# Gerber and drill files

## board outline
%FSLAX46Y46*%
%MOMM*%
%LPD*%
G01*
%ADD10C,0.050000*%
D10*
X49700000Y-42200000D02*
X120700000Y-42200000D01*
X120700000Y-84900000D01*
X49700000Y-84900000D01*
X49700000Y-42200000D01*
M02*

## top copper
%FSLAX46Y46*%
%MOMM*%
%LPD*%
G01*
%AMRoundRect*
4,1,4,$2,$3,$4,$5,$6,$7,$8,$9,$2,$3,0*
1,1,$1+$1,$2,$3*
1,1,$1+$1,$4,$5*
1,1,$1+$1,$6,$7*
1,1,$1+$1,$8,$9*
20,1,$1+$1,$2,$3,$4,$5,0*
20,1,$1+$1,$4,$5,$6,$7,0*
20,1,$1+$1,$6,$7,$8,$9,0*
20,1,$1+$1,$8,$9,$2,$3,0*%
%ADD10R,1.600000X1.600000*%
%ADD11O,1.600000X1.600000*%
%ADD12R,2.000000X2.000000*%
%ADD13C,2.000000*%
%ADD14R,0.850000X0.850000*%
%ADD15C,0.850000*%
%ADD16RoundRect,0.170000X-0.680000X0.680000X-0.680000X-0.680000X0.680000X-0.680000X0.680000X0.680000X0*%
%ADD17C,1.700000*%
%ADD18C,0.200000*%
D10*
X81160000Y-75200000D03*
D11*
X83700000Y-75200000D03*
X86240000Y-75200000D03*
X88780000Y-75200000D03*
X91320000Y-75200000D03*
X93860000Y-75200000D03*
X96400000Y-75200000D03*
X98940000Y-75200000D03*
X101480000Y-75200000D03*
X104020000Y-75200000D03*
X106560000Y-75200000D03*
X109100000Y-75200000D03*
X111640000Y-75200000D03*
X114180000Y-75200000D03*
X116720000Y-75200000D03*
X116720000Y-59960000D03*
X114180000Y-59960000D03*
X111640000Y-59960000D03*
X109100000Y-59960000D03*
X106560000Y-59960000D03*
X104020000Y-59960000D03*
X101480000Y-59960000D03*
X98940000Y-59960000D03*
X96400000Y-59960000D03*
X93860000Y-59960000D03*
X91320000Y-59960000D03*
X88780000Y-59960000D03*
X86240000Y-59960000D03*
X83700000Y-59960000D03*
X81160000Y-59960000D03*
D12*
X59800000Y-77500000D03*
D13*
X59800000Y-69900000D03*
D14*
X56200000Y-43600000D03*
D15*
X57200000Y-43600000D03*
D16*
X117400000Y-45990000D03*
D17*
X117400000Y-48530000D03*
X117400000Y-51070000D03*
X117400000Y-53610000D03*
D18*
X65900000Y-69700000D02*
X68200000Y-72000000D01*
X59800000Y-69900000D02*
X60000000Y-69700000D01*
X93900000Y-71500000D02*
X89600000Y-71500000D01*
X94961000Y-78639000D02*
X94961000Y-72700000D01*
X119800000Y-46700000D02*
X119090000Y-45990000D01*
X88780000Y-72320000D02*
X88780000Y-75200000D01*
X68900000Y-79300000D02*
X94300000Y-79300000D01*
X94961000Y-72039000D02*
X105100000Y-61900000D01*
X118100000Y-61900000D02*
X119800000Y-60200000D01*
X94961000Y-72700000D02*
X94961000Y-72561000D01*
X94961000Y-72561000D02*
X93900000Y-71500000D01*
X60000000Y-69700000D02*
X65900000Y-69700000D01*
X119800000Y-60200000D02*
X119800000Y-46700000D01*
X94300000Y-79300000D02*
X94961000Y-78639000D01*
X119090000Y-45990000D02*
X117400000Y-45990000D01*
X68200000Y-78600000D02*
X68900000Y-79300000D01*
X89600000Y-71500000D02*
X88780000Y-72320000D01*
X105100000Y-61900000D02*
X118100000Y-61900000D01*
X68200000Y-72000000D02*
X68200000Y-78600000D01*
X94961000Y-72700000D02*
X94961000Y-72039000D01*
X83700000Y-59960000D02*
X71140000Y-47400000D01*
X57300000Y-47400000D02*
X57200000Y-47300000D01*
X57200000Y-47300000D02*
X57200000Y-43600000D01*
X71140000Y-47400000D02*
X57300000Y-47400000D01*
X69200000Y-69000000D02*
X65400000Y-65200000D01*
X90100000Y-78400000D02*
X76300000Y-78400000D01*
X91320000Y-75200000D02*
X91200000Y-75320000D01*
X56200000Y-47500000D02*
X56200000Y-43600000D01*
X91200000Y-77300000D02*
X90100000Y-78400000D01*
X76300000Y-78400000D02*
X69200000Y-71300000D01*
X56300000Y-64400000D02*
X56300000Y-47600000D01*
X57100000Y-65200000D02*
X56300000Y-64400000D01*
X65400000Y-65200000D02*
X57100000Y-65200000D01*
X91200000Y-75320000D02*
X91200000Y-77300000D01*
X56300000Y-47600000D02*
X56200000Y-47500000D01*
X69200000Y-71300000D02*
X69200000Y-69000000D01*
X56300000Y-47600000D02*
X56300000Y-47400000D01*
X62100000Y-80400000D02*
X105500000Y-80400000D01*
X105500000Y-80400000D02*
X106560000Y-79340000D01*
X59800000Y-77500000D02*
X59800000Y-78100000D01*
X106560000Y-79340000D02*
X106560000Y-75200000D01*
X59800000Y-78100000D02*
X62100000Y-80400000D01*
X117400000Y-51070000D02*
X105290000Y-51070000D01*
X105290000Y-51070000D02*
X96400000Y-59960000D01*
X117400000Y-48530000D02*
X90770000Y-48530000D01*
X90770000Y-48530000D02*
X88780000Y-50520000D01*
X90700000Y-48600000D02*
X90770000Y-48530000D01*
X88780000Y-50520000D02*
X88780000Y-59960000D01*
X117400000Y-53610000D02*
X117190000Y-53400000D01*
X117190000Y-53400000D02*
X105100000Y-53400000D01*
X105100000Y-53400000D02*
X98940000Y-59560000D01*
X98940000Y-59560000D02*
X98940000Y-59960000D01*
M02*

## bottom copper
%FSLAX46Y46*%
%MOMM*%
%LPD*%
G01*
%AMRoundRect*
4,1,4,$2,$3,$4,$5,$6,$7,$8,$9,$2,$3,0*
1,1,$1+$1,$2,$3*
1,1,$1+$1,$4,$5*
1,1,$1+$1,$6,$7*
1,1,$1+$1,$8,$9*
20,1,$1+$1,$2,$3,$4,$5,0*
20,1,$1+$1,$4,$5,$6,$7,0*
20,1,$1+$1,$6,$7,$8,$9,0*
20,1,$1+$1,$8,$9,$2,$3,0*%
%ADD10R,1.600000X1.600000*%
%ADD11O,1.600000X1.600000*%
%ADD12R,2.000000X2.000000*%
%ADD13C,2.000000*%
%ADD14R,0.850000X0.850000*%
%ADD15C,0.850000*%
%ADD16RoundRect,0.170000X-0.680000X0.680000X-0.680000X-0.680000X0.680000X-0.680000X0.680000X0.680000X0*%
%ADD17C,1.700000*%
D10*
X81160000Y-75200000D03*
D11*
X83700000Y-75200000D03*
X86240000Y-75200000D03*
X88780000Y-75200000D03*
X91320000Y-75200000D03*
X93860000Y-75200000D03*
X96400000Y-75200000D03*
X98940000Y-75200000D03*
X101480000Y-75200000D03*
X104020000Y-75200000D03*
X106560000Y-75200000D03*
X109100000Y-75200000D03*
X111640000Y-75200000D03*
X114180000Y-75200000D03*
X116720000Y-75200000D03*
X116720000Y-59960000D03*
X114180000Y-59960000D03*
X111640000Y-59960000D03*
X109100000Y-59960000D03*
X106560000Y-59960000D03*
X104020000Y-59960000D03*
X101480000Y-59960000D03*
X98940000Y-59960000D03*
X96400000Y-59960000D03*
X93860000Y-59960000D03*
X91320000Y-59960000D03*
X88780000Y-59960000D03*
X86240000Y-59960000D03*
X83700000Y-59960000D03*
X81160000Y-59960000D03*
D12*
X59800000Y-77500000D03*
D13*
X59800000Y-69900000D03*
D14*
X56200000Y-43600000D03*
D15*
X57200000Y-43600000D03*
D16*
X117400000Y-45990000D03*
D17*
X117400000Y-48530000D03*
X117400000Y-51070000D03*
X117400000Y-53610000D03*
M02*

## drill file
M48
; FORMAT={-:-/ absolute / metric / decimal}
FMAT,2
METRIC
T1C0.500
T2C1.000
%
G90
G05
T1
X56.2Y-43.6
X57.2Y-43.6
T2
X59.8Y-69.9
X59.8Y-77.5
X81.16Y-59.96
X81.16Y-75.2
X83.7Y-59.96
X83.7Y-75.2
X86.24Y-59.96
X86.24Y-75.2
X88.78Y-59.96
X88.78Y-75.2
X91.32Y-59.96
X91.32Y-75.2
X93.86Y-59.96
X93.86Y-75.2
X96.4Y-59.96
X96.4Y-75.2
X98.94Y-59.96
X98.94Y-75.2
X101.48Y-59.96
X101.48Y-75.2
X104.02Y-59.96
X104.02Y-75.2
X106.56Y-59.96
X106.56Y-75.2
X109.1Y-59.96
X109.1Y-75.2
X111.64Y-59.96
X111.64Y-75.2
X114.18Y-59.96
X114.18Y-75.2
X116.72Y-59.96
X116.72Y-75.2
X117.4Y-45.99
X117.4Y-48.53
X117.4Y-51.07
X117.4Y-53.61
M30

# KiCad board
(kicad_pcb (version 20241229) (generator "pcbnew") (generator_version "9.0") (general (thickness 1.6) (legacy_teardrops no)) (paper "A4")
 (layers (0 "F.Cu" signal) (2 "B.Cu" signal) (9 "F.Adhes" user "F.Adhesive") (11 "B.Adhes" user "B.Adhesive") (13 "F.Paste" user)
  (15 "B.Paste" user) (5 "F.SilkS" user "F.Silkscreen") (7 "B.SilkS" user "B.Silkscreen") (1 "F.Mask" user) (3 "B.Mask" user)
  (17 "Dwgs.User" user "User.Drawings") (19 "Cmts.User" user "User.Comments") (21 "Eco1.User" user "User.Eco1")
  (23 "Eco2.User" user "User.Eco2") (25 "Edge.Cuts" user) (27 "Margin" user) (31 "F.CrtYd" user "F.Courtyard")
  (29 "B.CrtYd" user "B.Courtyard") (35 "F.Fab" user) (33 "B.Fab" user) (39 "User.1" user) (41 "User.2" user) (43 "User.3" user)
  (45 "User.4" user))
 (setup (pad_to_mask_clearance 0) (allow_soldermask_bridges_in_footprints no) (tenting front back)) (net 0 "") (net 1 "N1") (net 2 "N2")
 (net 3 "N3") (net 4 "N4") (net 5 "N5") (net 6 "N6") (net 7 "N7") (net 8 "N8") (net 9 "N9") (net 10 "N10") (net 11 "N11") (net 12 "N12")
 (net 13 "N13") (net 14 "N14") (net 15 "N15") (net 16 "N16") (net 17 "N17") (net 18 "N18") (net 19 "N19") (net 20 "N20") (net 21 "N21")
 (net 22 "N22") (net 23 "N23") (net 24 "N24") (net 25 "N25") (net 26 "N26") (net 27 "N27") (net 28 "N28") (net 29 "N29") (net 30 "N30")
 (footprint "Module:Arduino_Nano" (layer "F.Cu") (at 81.16 75.2 90)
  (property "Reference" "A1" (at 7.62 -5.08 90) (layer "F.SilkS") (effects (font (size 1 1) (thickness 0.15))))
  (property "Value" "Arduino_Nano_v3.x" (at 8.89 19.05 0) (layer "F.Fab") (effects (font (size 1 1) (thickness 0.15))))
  (pad "1" thru_hole rect (at 0 0 90) (size 1.6 1.6) (drill 1) (layers "*.Cu" "*.Mask") (remove_unused_layers no) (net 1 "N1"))
  (pad "2" thru_hole oval (at 0 2.54 90) (size 1.6 1.6) (drill 1) (layers "*.Cu" "*.Mask") (remove_unused_layers no) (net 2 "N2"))
  (pad "3" thru_hole oval (at 0 5.08 90) (size 1.6 1.6) (drill 1) (layers "*.Cu" "*.Mask") (remove_unused_layers no) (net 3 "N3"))
  (pad "4" thru_hole oval (at 0 7.62 90) (size 1.6 1.6) (drill 1) (layers "*.Cu" "*.Mask") (remove_unused_layers no) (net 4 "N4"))
  (pad "5" thru_hole oval (at 0 10.16 90) (size 1.6 1.6) (drill 1) (layers "*.Cu" "*.Mask") (remove_unused_layers no) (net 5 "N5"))
  (pad "6" thru_hole oval (at 0 12.7 90) (size 1.6 1.6) (drill 1) (layers "*.Cu" "*.Mask") (remove_unused_layers no) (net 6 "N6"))
  (pad "7" thru_hole oval (at 0 15.24 90) (size 1.6 1.6) (drill 1) (layers "*.Cu" "*.Mask") (remove_unused_layers no) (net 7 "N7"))
  (pad "8" thru_hole oval (at 0 17.78 90) (size 1.6 1.6) (drill 1) (layers "*.Cu" "*.Mask") (remove_unused_layers no) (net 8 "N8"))
  (pad "9" thru_hole oval (at 0 20.32 90) (size 1.6 1.6) (drill 1) (layers "*.Cu" "*.Mask") (remove_unused_layers no) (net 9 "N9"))
  (pad "10" thru_hole oval (at 0 22.86 90) (size 1.6 1.6) (drill 1) (layers "*.Cu" "*.Mask") (remove_unused_layers no) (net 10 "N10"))
  (pad "11" thru_hole oval (at 0 25.4 90) (size 1.6 1.6) (drill 1) (layers "*.Cu" "*.Mask") (remove_unused_layers no) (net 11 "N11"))
  (pad "12" thru_hole oval (at 0 27.94 90) (size 1.6 1.6) (drill 1) (layers "*.Cu" "*.Mask") (remove_unused_layers no) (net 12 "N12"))
  (pad "13" thru_hole oval (at 0 30.48 90) (size 1.6 1.6) (drill 1) (layers "*.Cu" "*.Mask") (remove_unused_layers no) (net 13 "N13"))
  (pad "14" thru_hole oval (at 0 33.02 90) (size 1.6 1.6) (drill 1) (layers "*.Cu" "*.Mask") (remove_unused_layers no) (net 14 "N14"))
  (pad "15" thru_hole oval (at 0 35.56 90) (size 1.6 1.6) (drill 1) (layers "*.Cu" "*.Mask") (remove_unused_layers no) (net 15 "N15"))
  (pad "16" thru_hole oval (at 15.24 35.56 90) (size 1.6 1.6) (drill 1) (layers "*.Cu" "*.Mask") (remove_unused_layers no) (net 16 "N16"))
  (pad "17" thru_hole oval (at 15.24 33.02 90) (size 1.6 1.6) (drill 1) (layers "*.Cu" "*.Mask") (remove_unused_layers no) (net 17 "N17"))
  (pad "18" thru_hole oval (at 15.24 30.48 90) (size 1.6 1.6) (drill 1) (layers "*.Cu" "*.Mask") (remove_unused_layers no) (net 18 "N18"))
  (pad "19" thru_hole oval (at 15.24 27.94 90) (size 1.6 1.6) (drill 1) (layers "*.Cu" "*.Mask") (remove_unused_layers no) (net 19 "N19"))
  (pad "20" thru_hole oval (at 15.24 25.4 90) (size 1.6 1.6) (drill 1) (layers "*.Cu" "*.Mask") (remove_unused_layers no) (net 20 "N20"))
  (pad "21" thru_hole oval (at 15.24 22.86 90) (size 1.6 1.6) (drill 1) (layers "*.Cu" "*.Mask") (remove_unused_layers no) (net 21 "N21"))
  (pad "22" thru_hole oval (at 15.24 20.32 90) (size 1.6 1.6) (drill 1) (layers "*.Cu" "*.Mask") (remove_unused_layers no) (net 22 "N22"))
  (pad "23" thru_hole oval (at 15.24 17.78 90) (size 1.6 1.6) (drill 1) (layers "*.Cu" "*.Mask") (remove_unused_layers no) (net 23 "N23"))
  (pad "24" thru_hole oval (at 15.24 15.24 90) (size 1.6 1.6) (drill 1) (layers "*.Cu" "*.Mask") (remove_unused_layers no) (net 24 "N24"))
  (pad "25" thru_hole oval (at 15.24 12.7 90) (size 1.6 1.6) (drill 1) (layers "*.Cu" "*.Mask") (remove_unused_layers no) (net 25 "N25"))
  (pad "26" thru_hole oval (at 15.24 10.16 90) (size 1.6 1.6) (drill 1) (layers "*.Cu" "*.Mask") (remove_unused_layers no) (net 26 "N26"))
  (pad "27" thru_hole oval (at 15.24 7.62 90) (size 1.6 1.6) (drill 1) (layers "*.Cu" "*.Mask") (remove_unused_layers no) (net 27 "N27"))
  (pad "28" thru_hole oval (at 15.24 5.08 90) (size 1.6 1.6) (drill 1) (layers "*.Cu" "*.Mask") (remove_unused_layers no) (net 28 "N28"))
  (pad "29" thru_hole oval (at 15.24 2.54 90) (size 1.6 1.6) (drill 1) (layers "*.Cu" "*.Mask") (remove_unused_layers no) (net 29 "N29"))
  (pad "30" thru_hole oval (at 15.24 0 90) (size 1.6 1.6) (drill 1) (layers "*.Cu" "*.Mask") (remove_unused_layers no) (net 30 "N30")))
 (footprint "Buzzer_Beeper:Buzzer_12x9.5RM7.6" (layer "F.Cu") (at 59.8 77.5 90)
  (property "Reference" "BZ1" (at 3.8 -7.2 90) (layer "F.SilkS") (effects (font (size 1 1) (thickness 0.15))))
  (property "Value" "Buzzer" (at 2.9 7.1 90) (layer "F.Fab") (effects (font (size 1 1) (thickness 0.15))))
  (pad "1" thru_hole rect (at 0 0 90) (size 2 2) (drill 1) (layers "*.Cu" "*.Mask") (remove_unused_layers no) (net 11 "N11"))
  (pad "2" thru_hole circle (at 7.6 0 90) (size 2 2) (drill 1) (layers "*.Cu" "*.Mask") (remove_unused_layers no) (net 4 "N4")))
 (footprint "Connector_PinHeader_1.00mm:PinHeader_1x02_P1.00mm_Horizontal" (layer "F.Cu") (at 56.2 43.6 90)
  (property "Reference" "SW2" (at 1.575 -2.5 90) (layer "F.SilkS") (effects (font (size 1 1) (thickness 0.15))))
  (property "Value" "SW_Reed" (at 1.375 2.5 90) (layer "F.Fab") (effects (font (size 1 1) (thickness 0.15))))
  (pad "1" thru_hole rect (at 0 0 90) (size 0.85 0.85) (drill 0.5) (layers "*.Cu" "*.Mask") (remove_unused_layers no) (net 5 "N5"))
  (pad "2" thru_hole circle (at 0 1 90) (size 0.85 0.85) (drill 0.5) (layers "*.Cu" "*.Mask") (remove_unused_layers no) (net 29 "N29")))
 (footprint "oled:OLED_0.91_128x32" (layer "F.Cu") (at 117.4 45.99 -90)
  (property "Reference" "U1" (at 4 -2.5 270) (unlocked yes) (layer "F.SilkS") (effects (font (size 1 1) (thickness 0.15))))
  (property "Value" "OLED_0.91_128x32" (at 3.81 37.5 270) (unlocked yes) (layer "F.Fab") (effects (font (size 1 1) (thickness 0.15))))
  (pad "1" thru_hole roundrect (at 0 0 270) (size 1.7 1.7) (drill 1) (layers "*.Cu" "*.Mask") (remove_unused_layers no)
   (roundrect_rratio 0.1) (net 4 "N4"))
  (pad "2" thru_hole circle (at 2.54 0 270) (size 1.7 1.7) (drill 1) (layers "*.Cu" "*.Mask") (remove_unused_layers no) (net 27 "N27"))
  (pad "3" thru_hole circle (at 5.08 0 270) (size 1.7 1.7) (drill 1) (layers "*.Cu" "*.Mask") (remove_unused_layers no) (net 24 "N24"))
  (pad "4" thru_hole circle (at 7.62 0 270) (size 1.7 1.7) (drill 1) (layers "*.Cu" "*.Mask") (remove_unused_layers no) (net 23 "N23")))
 (gr_rect (start 49.7 42.2) (end 120.7 84.9) (stroke (width 0.05) (type solid)) (fill no) (layer "Edge.Cuts"))
 (segment (start 65.9 69.7) (end 68.2 72) (width 0.2) (layer "F.Cu") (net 4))
 (segment (start 59.8 69.9) (end 60 69.7) (width 0.2) (layer "F.Cu") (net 4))
 (segment (start 93.9 71.5) (end 89.6 71.5) (width 0.2) (layer "F.Cu") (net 4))
 (segment (start 94.961 78.639) (end 94.961 72.7) (width 0.2) (layer "F.Cu") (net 4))
 (segment (start 119.8 46.7) (end 119.09 45.99) (width 0.2) (layer "F.Cu") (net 4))
 (segment (start 88.78 72.32) (end 88.78 75.2) (width 0.2) (layer "F.Cu") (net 4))
 (segment (start 68.9 79.3) (end 94.3 79.3) (width 0.2) (layer "F.Cu") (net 4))
 (segment (start 94.961 72.039) (end 105.1 61.9) (width 0.2) (layer "F.Cu") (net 4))
 (segment (start 118.1 61.9) (end 119.8 60.2) (width 0.2) (layer "F.Cu") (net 4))
 (segment (start 94.961 72.7) (end 94.961 72.561) (width 0.2) (layer "F.Cu") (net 4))
 (segment (start 94.961 72.561) (end 93.9 71.5) (width 0.2) (layer "F.Cu") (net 4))
 (segment (start 60 69.7) (end 65.9 69.7) (width 0.2) (layer "F.Cu") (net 4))
 (segment (start 119.8 60.2) (end 119.8 46.7) (width 0.2) (layer "F.Cu") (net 4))
 (segment (start 94.3 79.3) (end 94.961 78.639) (width 0.2) (layer "F.Cu") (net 4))
 (segment (start 119.09 45.99) (end 117.4 45.99) (width 0.2) (layer "F.Cu") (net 4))
 (segment (start 68.2 78.6) (end 68.9 79.3) (width 0.2) (layer "F.Cu") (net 4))
 (segment (start 89.6 71.5) (end 88.78 72.32) (width 0.2) (layer "F.Cu") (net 4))
 (segment (start 105.1 61.9) (end 118.1 61.9) (width 0.2) (layer "F.Cu") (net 4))
 (segment (start 68.2 72) (end 68.2 78.6) (width 0.2) (layer "F.Cu") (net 4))
 (segment (start 94.961 72.7) (end 94.961 72.039) (width 0.2) (layer "F.Cu") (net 4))
 (segment (start 83.7 59.96) (end 71.14 47.4) (width 0.2) (layer "F.Cu") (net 29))
 (segment (start 57.3 47.4) (end 57.2 47.3) (width 0.2) (layer "F.Cu") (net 29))
 (segment (start 57.2 47.3) (end 57.2 43.6) (width 0.2) (layer "F.Cu") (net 29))
 (segment (start 71.14 47.4) (end 57.3 47.4) (width 0.2) (layer "F.Cu") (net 29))
 (segment (start 69.2 69) (end 65.4 65.2) (width 0.2) (layer "F.Cu") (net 5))
 (segment (start 90.1 78.4) (end 76.3 78.4) (width 0.2) (layer "F.Cu") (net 5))
 (segment (start 91.32 75.2) (end 91.2 75.32) (width 0.2) (layer "F.Cu") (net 5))
 (segment (start 56.2 47.5) (end 56.2 43.6) (width 0.2) (layer "F.Cu") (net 5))
 (segment (start 91.2 77.3) (end 90.1 78.4) (width 0.2) (layer "F.Cu") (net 5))
 (segment (start 76.3 78.4) (end 69.2 71.3) (width 0.2) (layer "F.Cu") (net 5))
 (segment (start 56.3 64.4) (end 56.3 47.6) (width 0.2) (layer "F.Cu") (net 5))
 (segment (start 57.1 65.2) (end 56.3 64.4) (width 0.2) (layer "F.Cu") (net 5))
 (segment (start 65.4 65.2) (end 57.1 65.2) (width 0.2) (layer "F.Cu") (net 5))
 (segment (start 91.2 75.32) (end 91.2 77.3) (width 0.2) (layer "F.Cu") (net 5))
 (segment (start 56.3 47.6) (end 56.2 47.5) (width 0.2) (layer "F.Cu") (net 5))
 (segment (start 69.2 71.3) (end 69.2 69) (width 0.2) (layer "F.Cu") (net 5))
 (segment (start 56.3 47.6) (end 56.3 47.4) (width 0.2) (layer "F.Cu") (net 5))
 (segment (start 62.1 80.4) (end 105.5 80.4) (width 0.2) (layer "F.Cu") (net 11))
 (segment (start 105.5 80.4) (end 106.56 79.34) (width 0.2) (layer "F.Cu") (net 11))
 (segment (start 59.8 77.5) (end 59.8 78.1) (width 0.2) (layer "F.Cu") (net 11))
 (segment (start 106.56 79.34) (end 106.56 75.2) (width 0.2) (layer "F.Cu") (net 11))
 (segment (start 59.8 78.1) (end 62.1 80.4) (width 0.2) (layer "F.Cu") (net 11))
 (segment (start 117.4 51.07) (end 105.29 51.07) (width 0.2) (layer "F.Cu") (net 24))
 (segment (start 105.29 51.07) (end 96.4 59.96) (width 0.2) (layer "F.Cu") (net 24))
 (segment (start 117.4 48.53) (end 90.77 48.53) (width 0.2) (layer "F.Cu") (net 27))
 (segment (start 90.77 48.53) (end 88.78 50.52) (width 0.2) (layer "F.Cu") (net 27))
 (segment (start 90.7 48.6) (end 90.77 48.53) (width 0.2) (layer "F.Cu") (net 27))
 (segment (start 88.78 50.52) (end 88.78 59.96) (width 0.2) (layer "F.Cu") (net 27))
 (segment (start 117.4 53.61) (end 117.19 53.4) (width 0.2) (layer "F.Cu") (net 23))
 (segment (start 117.19 53.4) (end 105.1 53.4) (width 0.2) (layer "F.Cu") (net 23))
 (segment (start 105.1 53.4) (end 98.94 59.56) (width 0.2) (layer "F.Cu") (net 23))
 (segment (start 98.94 59.56) (end 98.94 59.96) (width 0.2) (layer "F.Cu") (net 23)))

